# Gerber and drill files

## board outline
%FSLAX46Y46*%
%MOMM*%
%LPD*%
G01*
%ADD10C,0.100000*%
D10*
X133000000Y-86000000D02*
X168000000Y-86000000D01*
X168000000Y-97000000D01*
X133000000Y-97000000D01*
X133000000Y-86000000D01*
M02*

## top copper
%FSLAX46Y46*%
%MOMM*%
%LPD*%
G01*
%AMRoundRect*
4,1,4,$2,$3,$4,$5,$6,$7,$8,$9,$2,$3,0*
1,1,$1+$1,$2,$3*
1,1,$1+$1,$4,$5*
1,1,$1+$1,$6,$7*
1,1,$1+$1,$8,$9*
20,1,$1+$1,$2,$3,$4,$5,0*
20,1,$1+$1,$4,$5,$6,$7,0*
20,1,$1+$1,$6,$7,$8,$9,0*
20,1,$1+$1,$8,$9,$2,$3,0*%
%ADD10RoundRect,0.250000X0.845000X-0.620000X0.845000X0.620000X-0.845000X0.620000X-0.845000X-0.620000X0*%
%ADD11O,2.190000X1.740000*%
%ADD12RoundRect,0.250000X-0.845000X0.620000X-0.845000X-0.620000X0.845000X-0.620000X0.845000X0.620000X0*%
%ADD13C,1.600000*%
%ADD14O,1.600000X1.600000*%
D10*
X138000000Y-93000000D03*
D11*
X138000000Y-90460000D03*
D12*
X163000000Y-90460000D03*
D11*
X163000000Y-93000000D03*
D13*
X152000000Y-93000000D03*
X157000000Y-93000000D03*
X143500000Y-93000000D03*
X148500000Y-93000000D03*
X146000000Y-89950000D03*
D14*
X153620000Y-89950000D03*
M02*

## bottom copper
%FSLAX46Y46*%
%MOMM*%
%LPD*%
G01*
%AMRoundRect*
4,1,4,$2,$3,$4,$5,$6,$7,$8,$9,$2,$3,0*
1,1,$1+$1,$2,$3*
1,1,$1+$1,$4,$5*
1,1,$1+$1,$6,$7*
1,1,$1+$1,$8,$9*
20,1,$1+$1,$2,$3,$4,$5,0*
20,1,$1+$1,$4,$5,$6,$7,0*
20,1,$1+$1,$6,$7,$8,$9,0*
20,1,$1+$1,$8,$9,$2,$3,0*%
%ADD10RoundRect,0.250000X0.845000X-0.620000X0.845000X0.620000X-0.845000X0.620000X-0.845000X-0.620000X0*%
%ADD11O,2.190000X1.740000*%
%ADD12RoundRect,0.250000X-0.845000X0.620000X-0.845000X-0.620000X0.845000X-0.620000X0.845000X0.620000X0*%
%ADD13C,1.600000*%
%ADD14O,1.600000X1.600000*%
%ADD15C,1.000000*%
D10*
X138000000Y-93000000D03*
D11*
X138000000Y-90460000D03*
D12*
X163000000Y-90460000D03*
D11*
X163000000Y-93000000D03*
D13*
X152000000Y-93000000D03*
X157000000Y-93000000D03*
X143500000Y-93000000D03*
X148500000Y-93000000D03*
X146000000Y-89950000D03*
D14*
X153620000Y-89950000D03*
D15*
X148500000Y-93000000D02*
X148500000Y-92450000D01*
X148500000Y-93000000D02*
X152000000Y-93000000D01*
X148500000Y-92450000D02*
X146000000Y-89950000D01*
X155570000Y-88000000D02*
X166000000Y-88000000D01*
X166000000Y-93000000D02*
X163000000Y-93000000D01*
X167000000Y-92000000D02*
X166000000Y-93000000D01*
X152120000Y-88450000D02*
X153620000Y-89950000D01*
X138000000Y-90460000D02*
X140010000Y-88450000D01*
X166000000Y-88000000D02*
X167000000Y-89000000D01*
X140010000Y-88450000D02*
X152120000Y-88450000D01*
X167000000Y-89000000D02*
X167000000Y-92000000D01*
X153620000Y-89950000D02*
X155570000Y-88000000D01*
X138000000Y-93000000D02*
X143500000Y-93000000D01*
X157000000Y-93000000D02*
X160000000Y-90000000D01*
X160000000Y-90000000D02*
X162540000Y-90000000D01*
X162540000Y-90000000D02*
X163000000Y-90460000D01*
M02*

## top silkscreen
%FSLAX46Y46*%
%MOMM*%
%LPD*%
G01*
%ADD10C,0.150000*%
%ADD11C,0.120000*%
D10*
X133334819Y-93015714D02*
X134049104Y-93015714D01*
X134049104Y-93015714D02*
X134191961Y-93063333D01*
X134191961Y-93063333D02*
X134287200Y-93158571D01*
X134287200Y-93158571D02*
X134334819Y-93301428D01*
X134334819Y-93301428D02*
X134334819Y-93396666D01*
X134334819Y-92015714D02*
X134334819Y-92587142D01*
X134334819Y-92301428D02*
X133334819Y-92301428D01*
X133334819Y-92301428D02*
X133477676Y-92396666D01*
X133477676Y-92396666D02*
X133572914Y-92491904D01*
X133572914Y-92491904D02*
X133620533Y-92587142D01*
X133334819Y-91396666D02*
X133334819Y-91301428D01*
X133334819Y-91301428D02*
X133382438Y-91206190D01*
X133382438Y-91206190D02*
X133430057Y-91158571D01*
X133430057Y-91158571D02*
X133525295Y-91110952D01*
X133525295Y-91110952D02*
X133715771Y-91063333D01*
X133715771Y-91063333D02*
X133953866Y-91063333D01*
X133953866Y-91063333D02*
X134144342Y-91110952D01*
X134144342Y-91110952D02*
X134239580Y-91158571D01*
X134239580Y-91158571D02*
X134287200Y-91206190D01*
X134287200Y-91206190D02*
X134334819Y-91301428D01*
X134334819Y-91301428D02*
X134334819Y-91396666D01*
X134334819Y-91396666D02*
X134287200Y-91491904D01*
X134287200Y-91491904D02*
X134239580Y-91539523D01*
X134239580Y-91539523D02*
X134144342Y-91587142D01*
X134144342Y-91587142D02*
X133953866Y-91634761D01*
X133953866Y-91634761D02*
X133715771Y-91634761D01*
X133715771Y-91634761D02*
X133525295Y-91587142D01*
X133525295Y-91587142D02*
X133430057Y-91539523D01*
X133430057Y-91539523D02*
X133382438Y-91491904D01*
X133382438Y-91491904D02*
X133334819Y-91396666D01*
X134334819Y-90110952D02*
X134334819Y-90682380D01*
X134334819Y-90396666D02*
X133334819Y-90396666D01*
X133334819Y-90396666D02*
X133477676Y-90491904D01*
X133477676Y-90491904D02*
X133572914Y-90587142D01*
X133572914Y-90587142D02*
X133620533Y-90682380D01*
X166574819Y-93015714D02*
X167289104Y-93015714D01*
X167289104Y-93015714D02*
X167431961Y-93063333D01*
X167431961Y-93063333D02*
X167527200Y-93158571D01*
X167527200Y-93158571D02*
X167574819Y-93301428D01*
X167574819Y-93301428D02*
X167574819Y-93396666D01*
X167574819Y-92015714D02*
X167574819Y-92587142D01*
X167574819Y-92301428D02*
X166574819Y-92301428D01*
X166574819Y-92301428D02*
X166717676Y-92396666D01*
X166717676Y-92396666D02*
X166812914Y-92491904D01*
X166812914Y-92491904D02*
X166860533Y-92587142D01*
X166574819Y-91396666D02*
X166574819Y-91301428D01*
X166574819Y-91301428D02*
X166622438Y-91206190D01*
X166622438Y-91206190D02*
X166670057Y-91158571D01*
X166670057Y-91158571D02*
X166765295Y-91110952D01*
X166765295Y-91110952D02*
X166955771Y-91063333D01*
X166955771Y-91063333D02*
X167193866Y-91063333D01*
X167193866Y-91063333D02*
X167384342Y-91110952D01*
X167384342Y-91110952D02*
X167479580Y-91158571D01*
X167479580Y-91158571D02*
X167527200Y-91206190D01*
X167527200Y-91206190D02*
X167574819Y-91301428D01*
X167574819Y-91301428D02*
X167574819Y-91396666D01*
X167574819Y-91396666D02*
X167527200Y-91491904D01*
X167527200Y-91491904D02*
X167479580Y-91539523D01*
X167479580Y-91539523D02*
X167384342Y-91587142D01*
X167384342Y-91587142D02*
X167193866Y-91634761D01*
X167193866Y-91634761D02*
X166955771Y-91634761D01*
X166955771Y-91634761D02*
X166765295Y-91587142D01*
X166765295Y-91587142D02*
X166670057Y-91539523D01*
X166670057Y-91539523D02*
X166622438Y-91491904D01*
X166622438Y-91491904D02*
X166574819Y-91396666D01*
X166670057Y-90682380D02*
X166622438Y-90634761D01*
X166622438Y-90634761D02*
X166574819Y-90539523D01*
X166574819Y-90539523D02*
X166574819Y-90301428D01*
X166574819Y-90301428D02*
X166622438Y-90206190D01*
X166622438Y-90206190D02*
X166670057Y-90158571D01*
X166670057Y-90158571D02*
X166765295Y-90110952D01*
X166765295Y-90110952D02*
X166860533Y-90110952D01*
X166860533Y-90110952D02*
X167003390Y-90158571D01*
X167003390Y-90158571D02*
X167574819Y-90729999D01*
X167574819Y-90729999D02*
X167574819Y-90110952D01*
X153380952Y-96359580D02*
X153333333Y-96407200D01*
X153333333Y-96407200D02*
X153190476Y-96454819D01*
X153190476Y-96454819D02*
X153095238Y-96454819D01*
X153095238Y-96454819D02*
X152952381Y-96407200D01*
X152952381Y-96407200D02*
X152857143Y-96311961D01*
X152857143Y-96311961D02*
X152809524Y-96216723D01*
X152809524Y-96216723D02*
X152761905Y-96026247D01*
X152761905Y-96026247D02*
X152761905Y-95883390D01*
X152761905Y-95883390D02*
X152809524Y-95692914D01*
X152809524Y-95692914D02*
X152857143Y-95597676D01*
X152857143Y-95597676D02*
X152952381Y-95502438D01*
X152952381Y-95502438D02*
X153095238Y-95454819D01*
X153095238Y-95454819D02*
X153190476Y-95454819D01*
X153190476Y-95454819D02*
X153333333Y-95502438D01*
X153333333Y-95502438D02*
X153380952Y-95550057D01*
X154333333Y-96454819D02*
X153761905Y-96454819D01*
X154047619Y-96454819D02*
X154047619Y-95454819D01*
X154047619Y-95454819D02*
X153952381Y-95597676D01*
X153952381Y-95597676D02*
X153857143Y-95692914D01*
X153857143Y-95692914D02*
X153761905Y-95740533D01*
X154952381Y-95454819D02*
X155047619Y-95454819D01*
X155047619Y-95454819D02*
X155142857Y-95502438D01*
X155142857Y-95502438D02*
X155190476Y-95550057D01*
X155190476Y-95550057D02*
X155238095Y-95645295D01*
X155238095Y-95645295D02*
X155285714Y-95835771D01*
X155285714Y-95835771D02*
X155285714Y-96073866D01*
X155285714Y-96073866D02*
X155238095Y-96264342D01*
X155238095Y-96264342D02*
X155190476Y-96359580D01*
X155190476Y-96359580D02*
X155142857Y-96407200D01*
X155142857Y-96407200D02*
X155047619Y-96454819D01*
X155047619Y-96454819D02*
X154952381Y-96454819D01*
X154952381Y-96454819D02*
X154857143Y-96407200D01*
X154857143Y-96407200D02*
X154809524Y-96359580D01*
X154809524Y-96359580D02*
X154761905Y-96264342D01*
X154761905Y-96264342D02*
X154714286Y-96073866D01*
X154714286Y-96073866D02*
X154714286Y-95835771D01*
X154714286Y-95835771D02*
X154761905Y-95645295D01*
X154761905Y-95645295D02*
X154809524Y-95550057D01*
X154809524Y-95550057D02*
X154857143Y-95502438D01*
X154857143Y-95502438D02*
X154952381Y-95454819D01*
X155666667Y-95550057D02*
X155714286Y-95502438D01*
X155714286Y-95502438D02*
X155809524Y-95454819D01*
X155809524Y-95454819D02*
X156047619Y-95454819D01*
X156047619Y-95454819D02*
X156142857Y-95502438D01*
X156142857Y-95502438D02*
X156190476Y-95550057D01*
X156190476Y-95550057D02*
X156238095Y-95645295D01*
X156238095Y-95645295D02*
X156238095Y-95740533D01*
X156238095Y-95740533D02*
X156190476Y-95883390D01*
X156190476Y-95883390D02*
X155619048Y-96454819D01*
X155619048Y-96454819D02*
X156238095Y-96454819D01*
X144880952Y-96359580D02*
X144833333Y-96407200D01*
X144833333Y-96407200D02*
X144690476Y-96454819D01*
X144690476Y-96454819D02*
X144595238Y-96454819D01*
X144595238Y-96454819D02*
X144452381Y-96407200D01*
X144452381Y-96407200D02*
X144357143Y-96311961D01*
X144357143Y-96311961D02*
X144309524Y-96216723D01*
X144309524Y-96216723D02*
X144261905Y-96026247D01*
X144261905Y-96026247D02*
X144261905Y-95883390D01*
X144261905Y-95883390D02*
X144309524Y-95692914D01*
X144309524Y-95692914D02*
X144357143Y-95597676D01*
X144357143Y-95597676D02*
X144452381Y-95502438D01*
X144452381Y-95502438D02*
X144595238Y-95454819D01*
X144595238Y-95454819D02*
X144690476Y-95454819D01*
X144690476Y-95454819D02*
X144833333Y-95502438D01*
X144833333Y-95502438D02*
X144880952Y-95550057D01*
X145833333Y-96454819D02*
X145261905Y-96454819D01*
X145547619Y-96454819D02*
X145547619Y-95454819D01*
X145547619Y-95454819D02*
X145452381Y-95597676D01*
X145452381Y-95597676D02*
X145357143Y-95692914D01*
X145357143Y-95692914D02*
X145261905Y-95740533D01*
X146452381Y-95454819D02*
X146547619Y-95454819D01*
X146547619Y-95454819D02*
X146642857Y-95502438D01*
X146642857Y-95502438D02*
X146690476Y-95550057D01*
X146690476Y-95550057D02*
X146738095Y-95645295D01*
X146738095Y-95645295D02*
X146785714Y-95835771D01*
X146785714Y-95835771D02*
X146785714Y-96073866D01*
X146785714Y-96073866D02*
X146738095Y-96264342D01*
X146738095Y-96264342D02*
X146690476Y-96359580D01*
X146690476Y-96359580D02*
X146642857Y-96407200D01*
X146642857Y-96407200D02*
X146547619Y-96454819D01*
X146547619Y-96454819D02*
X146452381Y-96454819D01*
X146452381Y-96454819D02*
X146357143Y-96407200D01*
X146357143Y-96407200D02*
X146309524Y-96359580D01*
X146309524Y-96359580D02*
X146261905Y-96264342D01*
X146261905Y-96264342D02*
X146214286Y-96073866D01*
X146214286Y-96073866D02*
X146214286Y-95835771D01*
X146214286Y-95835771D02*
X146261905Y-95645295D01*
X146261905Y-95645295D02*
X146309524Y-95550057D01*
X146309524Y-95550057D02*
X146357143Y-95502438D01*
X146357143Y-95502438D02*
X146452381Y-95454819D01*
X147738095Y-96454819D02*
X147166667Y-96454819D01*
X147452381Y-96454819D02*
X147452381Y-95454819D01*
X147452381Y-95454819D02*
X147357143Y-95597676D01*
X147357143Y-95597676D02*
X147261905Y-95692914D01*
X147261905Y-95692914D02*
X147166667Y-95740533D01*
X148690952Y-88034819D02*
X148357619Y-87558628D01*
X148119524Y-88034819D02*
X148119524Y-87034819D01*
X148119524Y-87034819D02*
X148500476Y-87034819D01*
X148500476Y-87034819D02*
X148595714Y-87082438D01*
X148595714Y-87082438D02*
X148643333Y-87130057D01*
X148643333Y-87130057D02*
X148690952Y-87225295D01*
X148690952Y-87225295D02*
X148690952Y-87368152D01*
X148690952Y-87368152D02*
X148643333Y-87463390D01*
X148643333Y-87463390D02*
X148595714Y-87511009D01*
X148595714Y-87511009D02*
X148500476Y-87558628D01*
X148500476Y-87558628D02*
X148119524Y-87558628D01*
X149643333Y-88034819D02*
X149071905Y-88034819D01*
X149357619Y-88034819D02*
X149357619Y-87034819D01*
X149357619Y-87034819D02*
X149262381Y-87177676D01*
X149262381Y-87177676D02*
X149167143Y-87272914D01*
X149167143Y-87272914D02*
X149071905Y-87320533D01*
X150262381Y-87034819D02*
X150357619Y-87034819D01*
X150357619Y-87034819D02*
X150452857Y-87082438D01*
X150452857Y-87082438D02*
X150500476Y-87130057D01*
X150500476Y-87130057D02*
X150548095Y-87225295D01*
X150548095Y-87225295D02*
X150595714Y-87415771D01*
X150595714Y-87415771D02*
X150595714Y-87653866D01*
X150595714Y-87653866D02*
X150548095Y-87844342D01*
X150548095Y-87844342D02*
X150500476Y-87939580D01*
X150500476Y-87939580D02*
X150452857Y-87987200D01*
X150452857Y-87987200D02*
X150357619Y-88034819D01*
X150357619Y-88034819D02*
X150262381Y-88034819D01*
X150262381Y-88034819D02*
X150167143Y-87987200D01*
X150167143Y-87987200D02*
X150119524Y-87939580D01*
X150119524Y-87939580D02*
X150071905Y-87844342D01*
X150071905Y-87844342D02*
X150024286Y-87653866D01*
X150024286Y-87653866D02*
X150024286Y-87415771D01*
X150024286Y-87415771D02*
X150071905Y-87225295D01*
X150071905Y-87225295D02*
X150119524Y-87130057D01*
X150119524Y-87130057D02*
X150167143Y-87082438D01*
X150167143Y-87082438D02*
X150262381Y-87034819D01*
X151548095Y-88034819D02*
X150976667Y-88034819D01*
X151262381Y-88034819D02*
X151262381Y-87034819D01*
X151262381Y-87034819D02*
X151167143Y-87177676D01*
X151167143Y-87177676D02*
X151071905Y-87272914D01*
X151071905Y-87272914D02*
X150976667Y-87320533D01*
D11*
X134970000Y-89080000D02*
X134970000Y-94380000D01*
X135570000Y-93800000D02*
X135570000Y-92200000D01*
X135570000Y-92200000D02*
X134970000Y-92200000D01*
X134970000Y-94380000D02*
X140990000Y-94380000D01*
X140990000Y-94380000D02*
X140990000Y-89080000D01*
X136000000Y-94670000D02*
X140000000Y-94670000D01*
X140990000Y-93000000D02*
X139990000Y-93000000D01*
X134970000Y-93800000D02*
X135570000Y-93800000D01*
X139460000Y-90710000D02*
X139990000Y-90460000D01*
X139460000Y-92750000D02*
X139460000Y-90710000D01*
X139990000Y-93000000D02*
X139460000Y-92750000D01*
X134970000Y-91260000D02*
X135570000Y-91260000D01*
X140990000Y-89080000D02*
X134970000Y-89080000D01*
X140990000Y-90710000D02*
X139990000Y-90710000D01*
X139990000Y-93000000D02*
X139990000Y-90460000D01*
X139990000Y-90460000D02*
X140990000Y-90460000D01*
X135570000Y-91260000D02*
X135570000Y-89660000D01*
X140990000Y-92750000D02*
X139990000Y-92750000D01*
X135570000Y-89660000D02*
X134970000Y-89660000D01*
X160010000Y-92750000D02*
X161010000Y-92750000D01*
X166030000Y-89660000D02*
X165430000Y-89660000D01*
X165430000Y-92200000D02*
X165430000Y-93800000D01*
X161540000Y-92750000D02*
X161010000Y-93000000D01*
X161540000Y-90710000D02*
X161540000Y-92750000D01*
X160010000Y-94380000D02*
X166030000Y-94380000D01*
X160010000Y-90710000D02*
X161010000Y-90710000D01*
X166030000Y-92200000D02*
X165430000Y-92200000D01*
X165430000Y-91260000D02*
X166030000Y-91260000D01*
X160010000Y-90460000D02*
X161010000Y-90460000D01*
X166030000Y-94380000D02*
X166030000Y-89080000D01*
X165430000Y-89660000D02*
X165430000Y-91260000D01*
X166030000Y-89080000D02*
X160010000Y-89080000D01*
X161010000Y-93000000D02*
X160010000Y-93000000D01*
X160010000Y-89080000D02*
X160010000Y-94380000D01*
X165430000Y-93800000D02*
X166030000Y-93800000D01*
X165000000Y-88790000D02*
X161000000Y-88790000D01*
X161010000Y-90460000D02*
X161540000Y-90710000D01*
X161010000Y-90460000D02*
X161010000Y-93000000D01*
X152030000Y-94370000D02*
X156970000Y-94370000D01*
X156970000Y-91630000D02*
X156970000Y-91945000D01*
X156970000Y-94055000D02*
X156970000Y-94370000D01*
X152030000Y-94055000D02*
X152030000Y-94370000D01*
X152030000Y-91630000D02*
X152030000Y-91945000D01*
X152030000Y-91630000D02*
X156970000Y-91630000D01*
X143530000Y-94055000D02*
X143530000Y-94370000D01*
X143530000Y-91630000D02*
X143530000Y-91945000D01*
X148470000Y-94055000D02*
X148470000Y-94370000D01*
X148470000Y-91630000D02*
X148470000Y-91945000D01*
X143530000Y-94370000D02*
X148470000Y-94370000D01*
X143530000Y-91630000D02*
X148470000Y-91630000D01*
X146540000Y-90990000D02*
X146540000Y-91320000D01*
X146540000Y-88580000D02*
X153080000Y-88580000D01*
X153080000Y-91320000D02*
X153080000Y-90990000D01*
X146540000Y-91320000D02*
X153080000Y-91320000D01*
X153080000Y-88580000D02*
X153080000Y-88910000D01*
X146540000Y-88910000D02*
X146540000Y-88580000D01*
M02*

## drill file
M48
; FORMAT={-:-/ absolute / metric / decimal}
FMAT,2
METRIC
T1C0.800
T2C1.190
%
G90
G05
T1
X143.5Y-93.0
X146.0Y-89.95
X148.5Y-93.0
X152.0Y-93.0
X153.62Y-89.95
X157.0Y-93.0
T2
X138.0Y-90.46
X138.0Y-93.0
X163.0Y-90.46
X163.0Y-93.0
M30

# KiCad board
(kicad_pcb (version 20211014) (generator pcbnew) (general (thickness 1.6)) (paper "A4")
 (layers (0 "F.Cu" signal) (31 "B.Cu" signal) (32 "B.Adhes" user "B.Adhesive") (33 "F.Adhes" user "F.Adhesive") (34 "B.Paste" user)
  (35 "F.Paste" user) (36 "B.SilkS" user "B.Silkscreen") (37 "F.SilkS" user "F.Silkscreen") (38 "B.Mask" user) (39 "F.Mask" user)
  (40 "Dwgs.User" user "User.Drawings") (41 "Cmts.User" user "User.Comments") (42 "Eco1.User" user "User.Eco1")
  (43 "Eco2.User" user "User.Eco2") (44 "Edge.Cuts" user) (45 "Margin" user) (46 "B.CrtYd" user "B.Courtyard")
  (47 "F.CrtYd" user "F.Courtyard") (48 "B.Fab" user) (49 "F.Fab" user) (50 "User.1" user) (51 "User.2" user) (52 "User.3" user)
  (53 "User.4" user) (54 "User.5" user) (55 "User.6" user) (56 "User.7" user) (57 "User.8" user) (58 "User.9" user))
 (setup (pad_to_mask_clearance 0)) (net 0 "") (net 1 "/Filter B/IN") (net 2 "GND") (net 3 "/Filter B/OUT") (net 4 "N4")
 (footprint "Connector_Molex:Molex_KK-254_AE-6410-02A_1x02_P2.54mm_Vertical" (layer "F.Cu") (at 138 93 90)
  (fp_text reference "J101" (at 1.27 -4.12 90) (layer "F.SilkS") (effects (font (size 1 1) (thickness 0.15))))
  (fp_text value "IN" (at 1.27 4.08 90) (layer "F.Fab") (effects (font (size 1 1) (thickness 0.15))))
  (fp_line (start 3.92 -3.03) (end -1.38 -3.03) (layer "F.SilkS") (width 0.12))
  (fp_line (start -0.8 -2.43) (end 0.8 -2.43) (layer "F.SilkS") (width 0.12))
  (fp_line (start 0.8 -2.43) (end 0.8 -3.03) (layer "F.SilkS") (width 0.12))
  (fp_line (start -1.38 -3.03) (end -1.38 2.99) (layer "F.SilkS") (width 0.12))
  (fp_line (start -1.38 2.99) (end 3.92 2.99) (layer "F.SilkS") (width 0.12))
  (fp_line (start -1.67 -2) (end -1.67 2) (layer "F.SilkS") (width 0.12))
  (fp_line (start 0 2.99) (end 0 1.99) (layer "F.SilkS") (width 0.12))
  (fp_line (start -0.8 -3.03) (end -0.8 -2.43) (layer "F.SilkS") (width 0.12))
  (fp_line (start 2.29 1.46) (end 2.54 1.99) (layer "F.SilkS") (width 0.12))
  (fp_line (start 0.25 1.46) (end 2.29 1.46) (layer "F.SilkS") (width 0.12))
  (fp_line (start 0 1.99) (end 0.25 1.46) (layer "F.SilkS") (width 0.12))
  (fp_line (start 1.74 -3.03) (end 1.74 -2.43) (layer "F.SilkS") (width 0.12))
  (fp_line (start 3.92 2.99) (end 3.92 -3.03) (layer "F.SilkS") (width 0.12))
  (fp_line (start 2.29 2.99) (end 2.29 1.99) (layer "F.SilkS") (width 0.12))
  (fp_line (start 0 1.99) (end 2.54 1.99) (layer "F.SilkS") (width 0.12))
  (fp_line (start 2.54 1.99) (end 2.54 2.99) (layer "F.SilkS") (width 0.12))
  (fp_line (start 1.74 -2.43) (end 3.34 -2.43) (layer "F.SilkS") (width 0.12))
  (fp_line (start 0.25 2.99) (end 0.25 1.99) (layer "F.SilkS") (width 0.12))
  (fp_line (start 3.34 -2.43) (end 3.34 -3.03) (layer "F.SilkS") (width 0.12))
  (pad "1" thru_hole roundrect (at 0 0 90) (size 1.74 2.19) (drill 1.19) (layers *.Cu *.Mask) (roundrect_rratio 0.143678)
   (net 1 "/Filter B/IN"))
  (pad "2" thru_hole oval (at 2.54 0 90) (size 1.74 2.19) (drill 1.19) (layers *.Cu *.Mask) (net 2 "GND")))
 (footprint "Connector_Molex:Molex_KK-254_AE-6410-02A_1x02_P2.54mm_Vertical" (layer "F.Cu") (at 163 90.46 -90)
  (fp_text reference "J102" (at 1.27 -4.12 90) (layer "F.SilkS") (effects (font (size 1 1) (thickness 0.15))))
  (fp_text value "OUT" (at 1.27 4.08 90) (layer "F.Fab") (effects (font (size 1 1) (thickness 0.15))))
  (fp_line (start 2.29 2.99) (end 2.29 1.99) (layer "F.SilkS") (width 0.12))
  (fp_line (start -0.8 -3.03) (end -0.8 -2.43) (layer "F.SilkS") (width 0.12))
  (fp_line (start 1.74 -2.43) (end 3.34 -2.43) (layer "F.SilkS") (width 0.12))
  (fp_line (start 2.29 1.46) (end 2.54 1.99) (layer "F.SilkS") (width 0.12))
  (fp_line (start 0.25 1.46) (end 2.29 1.46) (layer "F.SilkS") (width 0.12))
  (fp_line (start 3.92 2.99) (end 3.92 -3.03) (layer "F.SilkS") (width 0.12))
  (fp_line (start 0.25 2.99) (end 0.25 1.99) (layer "F.SilkS") (width 0.12))
  (fp_line (start 1.74 -3.03) (end 1.74 -2.43) (layer "F.SilkS") (width 0.12))
  (fp_line (start 0.8 -2.43) (end 0.8 -3.03) (layer "F.SilkS") (width 0.12))
  (fp_line (start 0 2.99) (end 0 1.99) (layer "F.SilkS") (width 0.12))
  (fp_line (start 3.92 -3.03) (end -1.38 -3.03) (layer "F.SilkS") (width 0.12))
  (fp_line (start -0.8 -2.43) (end 0.8 -2.43) (layer "F.SilkS") (width 0.12))
  (fp_line (start -1.38 -3.03) (end -1.38 2.99) (layer "F.SilkS") (width 0.12))
  (fp_line (start 2.54 1.99) (end 2.54 2.99) (layer "F.SilkS") (width 0.12))
  (fp_line (start -1.38 2.99) (end 3.92 2.99) (layer "F.SilkS") (width 0.12))
  (fp_line (start 3.34 -2.43) (end 3.34 -3.03) (layer "F.SilkS") (width 0.12))
  (fp_line (start -1.67 -2) (end -1.67 2) (layer "F.SilkS") (width 0.12))
  (fp_line (start 0 1.99) (end 0.25 1.46) (layer "F.SilkS") (width 0.12))
  (fp_line (start 0 1.99) (end 2.54 1.99) (layer "F.SilkS") (width 0.12))
  (pad "1" thru_hole roundrect (at 0 0 270) (size 1.74 2.19) (drill 1.19) (layers *.Cu *.Mask) (roundrect_rratio 0.143678)
   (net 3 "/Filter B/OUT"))
  (pad "2" thru_hole oval (at 2.54 0 270) (size 1.74 2.19) (drill 1.19) (layers *.Cu *.Mask) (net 2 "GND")))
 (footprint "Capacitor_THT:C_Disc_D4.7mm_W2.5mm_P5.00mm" (layer "F.Cu") (at 152 93)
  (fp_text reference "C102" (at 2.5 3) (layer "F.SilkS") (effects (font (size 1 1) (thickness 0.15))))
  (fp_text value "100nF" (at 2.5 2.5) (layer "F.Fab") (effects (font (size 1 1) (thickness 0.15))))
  (fp_line (start 0.03 1.37) (end 4.97 1.37) (layer "F.SilkS") (width 0.12))
  (fp_line (start 4.97 -1.37) (end 4.97 -1.055) (layer "F.SilkS") (width 0.12))
  (fp_line (start 4.97 1.055) (end 4.97 1.37) (layer "F.SilkS") (width 0.12))
  (fp_line (start 0.03 1.055) (end 0.03 1.37) (layer "F.SilkS") (width 0.12))
  (fp_line (start 0.03 -1.37) (end 0.03 -1.055) (layer "F.SilkS") (width 0.12))
  (fp_line (start 0.03 -1.37) (end 4.97 -1.37) (layer "F.SilkS") (width 0.12))
  (pad "1" thru_hole circle (at 0 0) (size 1.6 1.6) (drill 0.8) (layers *.Cu *.Mask) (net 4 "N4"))
  (pad "2" thru_hole circle (at 5 0) (size 1.6 1.6) (drill 0.8) (layers *.Cu *.Mask) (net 3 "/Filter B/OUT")))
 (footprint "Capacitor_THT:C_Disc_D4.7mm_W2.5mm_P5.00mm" (layer "F.Cu") (at 143.5 93)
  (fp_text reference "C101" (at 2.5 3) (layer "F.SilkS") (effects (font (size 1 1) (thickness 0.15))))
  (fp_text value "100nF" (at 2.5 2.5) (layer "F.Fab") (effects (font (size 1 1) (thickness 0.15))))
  (fp_line (start 0.03 1.055) (end 0.03 1.37) (layer "F.SilkS") (width 0.12))
  (fp_line (start 0.03 -1.37) (end 0.03 -1.055) (layer "F.SilkS") (width 0.12))
  (fp_line (start 4.97 1.055) (end 4.97 1.37) (layer "F.SilkS") (width 0.12))
  (fp_line (start 4.97 -1.37) (end 4.97 -1.055) (layer "F.SilkS") (width 0.12))
  (fp_line (start 0.03 1.37) (end 4.97 1.37) (layer "F.SilkS") (width 0.12))
  (fp_line (start 0.03 -1.37) (end 4.97 -1.37) (layer "F.SilkS") (width 0.12))
  (pad "1" thru_hole circle (at 0 0) (size 1.6 1.6) (drill 0.8) (layers *.Cu *.Mask) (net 1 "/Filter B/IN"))
  (pad "2" thru_hole circle (at 5 0) (size 1.6 1.6) (drill 0.8) (layers *.Cu *.Mask) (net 4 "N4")))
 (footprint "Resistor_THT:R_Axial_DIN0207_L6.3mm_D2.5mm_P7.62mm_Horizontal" (layer "F.Cu") (at 146 89.95)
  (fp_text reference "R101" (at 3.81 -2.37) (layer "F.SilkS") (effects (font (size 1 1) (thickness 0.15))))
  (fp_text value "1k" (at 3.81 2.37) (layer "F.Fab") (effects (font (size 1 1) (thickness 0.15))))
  (fp_line (start 0.54 1.04) (end 0.54 1.37) (layer "F.SilkS") (width 0.12))
  (fp_line (start 0.54 -1.37) (end 7.08 -1.37) (layer "F.SilkS") (width 0.12))
  (fp_line (start 7.08 1.37) (end 7.08 1.04) (layer "F.SilkS") (width 0.12))
  (fp_line (start 0.54 1.37) (end 7.08 1.37) (layer "F.SilkS") (width 0.12))
  (fp_line (start 7.08 -1.37) (end 7.08 -1.04) (layer "F.SilkS") (width 0.12))
  (fp_line (start 0.54 -1.04) (end 0.54 -1.37) (layer "F.SilkS") (width 0.12))
  (pad "1" thru_hole circle (at 0 0) (size 1.6 1.6) (drill 0.8) (layers *.Cu *.Mask) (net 4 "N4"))
  (pad "2" thru_hole oval (at 7.62 0) (size 1.6 1.6) (drill 0.8) (layers *.Cu *.Mask) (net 2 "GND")))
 (gr_rect (start 168 97) (end 133 86) (layer "Edge.Cuts") (width 0.1) (fill none))
 (segment (start 148.5 93) (end 148.5 92.45) (width 1) (layer "B.Cu") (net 4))
 (segment (start 148.5 93) (end 152 93) (width 1) (layer "B.Cu") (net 4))
 (segment (start 148.5 92.45) (end 146 89.95) (width 1) (layer "B.Cu") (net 4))
 (segment (start 155.57 88) (end 166 88) (width 1) (layer "B.Cu") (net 2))
 (segment (start 166 93) (end 163 93) (width 1) (layer "B.Cu") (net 2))
 (segment (start 167 92) (end 166 93) (width 1) (layer "B.Cu") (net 2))
 (segment (start 152.12 88.45) (end 153.62 89.95) (width 1) (layer "B.Cu") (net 2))
 (segment (start 138 90.46) (end 140.01 88.45) (width 1) (layer "B.Cu") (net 2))
 (segment (start 166 88) (end 167 89) (width 1) (layer "B.Cu") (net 2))
 (segment (start 140.01 88.45) (end 152.12 88.45) (width 1) (layer "B.Cu") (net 2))
 (segment (start 167 89) (end 167 92) (width 1) (layer "B.Cu") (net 2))
 (segment (start 153.62 89.95) (end 155.57 88) (width 1) (layer "B.Cu") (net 2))
 (segment (start 138 93) (end 143.5 93) (width 1) (layer "B.Cu") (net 1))
 (segment (start 157 93) (end 160 90) (width 1) (layer "B.Cu") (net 3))
 (segment (start 160 90) (end 162.54 90) (width 1) (layer "B.Cu") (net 3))
 (segment (start 162.54 90) (end 163 90.46) (width 1) (layer "B.Cu") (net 3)))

